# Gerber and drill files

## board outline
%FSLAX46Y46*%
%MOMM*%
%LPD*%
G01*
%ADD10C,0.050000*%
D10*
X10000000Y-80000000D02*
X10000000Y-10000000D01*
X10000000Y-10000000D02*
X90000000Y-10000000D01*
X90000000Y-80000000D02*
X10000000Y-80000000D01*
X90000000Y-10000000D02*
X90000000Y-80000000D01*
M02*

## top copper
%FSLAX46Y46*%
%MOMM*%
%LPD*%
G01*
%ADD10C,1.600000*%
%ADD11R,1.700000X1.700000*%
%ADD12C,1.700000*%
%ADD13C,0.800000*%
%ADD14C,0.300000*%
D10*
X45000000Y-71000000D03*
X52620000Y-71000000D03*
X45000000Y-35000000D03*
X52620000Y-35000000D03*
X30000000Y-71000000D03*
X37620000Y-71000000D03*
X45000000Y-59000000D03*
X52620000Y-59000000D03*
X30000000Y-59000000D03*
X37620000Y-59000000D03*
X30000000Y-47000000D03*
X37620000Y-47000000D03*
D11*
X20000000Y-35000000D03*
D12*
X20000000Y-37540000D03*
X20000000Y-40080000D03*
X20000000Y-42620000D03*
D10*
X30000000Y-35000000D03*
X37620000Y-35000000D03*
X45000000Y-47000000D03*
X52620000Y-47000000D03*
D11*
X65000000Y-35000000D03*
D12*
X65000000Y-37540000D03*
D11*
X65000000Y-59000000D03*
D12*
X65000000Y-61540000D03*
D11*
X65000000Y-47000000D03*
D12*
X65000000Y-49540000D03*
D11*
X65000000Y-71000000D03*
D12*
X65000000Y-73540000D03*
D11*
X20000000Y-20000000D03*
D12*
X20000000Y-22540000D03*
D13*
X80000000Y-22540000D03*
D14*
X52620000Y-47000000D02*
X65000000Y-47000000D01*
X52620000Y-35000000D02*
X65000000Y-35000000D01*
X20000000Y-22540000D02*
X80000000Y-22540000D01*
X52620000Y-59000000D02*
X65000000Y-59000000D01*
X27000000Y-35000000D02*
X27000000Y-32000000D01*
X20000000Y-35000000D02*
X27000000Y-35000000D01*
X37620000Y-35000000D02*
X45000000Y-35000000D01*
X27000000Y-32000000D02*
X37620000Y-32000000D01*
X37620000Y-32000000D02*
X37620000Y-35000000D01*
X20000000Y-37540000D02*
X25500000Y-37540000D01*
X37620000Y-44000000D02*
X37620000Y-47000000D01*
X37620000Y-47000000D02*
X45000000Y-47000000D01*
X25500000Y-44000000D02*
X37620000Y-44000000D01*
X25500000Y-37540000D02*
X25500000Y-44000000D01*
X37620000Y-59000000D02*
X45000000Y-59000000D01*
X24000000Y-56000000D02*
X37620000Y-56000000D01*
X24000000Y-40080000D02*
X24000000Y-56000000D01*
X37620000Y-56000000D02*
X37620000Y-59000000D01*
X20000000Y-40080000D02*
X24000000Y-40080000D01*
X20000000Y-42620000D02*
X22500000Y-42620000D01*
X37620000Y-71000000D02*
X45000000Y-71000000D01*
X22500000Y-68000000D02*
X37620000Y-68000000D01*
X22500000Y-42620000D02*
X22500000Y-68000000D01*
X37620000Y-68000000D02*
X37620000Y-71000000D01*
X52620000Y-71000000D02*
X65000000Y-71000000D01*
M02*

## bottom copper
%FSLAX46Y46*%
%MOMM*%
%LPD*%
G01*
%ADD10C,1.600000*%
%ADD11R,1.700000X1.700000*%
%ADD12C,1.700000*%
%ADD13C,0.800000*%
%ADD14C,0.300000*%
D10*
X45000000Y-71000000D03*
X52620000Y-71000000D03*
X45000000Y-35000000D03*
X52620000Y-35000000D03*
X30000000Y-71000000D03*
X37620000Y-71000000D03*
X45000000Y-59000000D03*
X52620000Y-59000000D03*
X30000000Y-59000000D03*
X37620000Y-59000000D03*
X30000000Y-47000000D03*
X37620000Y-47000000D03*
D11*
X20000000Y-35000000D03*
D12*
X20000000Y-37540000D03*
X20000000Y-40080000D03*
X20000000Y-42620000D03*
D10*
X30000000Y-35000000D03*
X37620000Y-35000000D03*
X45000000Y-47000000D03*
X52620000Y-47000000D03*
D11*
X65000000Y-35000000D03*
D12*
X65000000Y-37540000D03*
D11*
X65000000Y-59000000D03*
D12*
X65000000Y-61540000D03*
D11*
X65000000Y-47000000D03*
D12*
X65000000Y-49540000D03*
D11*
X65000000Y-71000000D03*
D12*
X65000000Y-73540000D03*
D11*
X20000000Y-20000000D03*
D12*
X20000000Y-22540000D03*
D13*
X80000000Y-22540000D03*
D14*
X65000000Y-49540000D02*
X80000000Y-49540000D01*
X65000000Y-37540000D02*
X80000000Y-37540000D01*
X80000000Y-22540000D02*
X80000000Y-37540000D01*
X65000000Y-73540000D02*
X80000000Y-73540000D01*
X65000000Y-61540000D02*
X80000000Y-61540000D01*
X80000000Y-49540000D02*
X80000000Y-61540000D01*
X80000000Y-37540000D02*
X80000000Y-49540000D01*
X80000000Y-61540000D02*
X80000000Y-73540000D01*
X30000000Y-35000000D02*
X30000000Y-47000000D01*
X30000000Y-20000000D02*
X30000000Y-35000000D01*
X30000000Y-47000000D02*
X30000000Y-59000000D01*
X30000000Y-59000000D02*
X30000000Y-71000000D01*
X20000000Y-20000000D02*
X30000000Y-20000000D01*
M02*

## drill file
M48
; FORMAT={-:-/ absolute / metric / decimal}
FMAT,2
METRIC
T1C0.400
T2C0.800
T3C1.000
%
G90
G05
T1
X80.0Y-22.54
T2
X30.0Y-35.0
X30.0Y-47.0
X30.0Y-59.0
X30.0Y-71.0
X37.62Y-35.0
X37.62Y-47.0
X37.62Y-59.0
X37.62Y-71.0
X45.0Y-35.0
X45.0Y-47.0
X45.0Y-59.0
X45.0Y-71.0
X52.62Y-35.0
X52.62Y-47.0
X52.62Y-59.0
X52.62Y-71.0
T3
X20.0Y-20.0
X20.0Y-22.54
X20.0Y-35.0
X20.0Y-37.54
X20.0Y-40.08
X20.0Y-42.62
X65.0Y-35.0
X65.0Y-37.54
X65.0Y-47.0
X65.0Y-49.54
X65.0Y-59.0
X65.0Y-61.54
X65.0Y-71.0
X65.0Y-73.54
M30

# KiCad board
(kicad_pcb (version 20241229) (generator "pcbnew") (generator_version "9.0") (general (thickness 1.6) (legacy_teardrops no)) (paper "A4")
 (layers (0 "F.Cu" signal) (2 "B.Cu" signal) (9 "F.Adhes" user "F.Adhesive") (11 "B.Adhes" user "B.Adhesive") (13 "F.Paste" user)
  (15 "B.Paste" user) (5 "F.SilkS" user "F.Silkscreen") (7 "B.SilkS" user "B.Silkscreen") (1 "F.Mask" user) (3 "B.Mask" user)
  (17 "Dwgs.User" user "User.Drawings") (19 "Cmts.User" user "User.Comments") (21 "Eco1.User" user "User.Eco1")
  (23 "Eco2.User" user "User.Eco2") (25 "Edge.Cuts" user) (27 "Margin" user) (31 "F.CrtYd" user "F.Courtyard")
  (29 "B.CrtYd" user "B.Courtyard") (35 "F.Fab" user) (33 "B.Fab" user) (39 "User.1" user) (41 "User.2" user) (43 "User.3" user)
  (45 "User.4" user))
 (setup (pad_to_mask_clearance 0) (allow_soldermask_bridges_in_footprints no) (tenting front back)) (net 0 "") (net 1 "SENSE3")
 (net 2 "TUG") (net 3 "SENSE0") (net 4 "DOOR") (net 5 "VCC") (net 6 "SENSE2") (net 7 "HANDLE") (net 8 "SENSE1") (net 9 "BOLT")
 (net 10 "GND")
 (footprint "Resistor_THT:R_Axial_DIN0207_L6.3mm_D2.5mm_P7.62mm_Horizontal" (layer "F.Cu") (at 45 71)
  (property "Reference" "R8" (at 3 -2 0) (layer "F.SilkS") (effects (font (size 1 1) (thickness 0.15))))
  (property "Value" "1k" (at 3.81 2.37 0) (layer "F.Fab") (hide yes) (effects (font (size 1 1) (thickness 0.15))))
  (pad "1" thru_hole circle (at 0 0) (size 1.6 1.6) (drill 0.8) (layers "*.Cu" "*.Mask") (remove_unused_layers no) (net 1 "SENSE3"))
  (pad "2" thru_hole circle (at 7.62 0) (size 1.6 1.6) (drill 0.8) (layers "*.Cu" "*.Mask") (remove_unused_layers no) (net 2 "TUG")))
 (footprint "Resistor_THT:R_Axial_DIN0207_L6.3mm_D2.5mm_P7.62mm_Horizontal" (layer "F.Cu") (at 45 35)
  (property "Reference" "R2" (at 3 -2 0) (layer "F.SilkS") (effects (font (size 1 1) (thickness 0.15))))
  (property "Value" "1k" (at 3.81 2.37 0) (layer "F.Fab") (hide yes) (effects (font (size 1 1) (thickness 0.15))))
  (pad "1" thru_hole circle (at 0 0) (size 1.6 1.6) (drill 0.8) (layers "*.Cu" "*.Mask") (remove_unused_layers no) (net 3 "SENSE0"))
  (pad "2" thru_hole circle (at 7.62 0) (size 1.6 1.6) (drill 0.8) (layers "*.Cu" "*.Mask") (remove_unused_layers no) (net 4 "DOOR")))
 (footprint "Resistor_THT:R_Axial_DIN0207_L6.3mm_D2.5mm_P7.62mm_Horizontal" (layer "F.Cu") (at 30 71)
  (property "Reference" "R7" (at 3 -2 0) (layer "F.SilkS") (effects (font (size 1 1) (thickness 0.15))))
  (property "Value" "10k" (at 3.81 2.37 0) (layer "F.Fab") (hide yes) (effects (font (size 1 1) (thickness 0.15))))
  (pad "1" thru_hole circle (at 0 0) (size 1.6 1.6) (drill 0.8) (layers "*.Cu" "*.Mask") (remove_unused_layers no) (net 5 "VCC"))
  (pad "2" thru_hole circle (at 7.62 0) (size 1.6 1.6) (drill 0.8) (layers "*.Cu" "*.Mask") (remove_unused_layers no) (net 1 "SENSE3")))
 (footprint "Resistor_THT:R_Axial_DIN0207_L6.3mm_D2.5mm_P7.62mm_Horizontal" (layer "F.Cu") (at 45 59)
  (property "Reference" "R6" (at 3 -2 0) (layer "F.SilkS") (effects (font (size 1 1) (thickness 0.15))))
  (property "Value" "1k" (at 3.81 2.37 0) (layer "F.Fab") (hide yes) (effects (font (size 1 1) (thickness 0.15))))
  (pad "1" thru_hole circle (at 0 0) (size 1.6 1.6) (drill 0.8) (layers "*.Cu" "*.Mask") (remove_unused_layers no) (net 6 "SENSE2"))
  (pad "2" thru_hole circle (at 7.62 0) (size 1.6 1.6) (drill 0.8) (layers "*.Cu" "*.Mask") (remove_unused_layers no) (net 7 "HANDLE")))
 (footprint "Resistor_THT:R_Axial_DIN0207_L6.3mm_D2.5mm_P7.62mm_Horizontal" (layer "F.Cu") (at 30 59)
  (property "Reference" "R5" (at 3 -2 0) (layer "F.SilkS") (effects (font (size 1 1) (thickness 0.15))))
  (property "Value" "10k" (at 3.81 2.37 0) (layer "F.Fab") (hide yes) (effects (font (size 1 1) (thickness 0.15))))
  (pad "1" thru_hole circle (at 0 0) (size 1.6 1.6) (drill 0.8) (layers "*.Cu" "*.Mask") (remove_unused_layers no) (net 5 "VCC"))
  (pad "2" thru_hole circle (at 7.62 0) (size 1.6 1.6) (drill 0.8) (layers "*.Cu" "*.Mask") (remove_unused_layers no) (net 6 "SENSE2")))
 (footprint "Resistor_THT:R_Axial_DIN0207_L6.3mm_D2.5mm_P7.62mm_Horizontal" (layer "F.Cu") (at 30 47)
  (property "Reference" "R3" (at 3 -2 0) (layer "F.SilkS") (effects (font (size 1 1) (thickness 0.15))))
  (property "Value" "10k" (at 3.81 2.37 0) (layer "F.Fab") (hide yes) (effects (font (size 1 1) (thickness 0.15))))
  (pad "1" thru_hole circle (at 0 0) (size 1.6 1.6) (drill 0.8) (layers "*.Cu" "*.Mask") (remove_unused_layers no) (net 5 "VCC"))
  (pad "2" thru_hole circle (at 7.62 0) (size 1.6 1.6) (drill 0.8) (layers "*.Cu" "*.Mask") (remove_unused_layers no) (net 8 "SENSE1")))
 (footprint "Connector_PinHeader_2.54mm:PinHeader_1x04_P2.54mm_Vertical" (layer "F.Cu") (at 20 35)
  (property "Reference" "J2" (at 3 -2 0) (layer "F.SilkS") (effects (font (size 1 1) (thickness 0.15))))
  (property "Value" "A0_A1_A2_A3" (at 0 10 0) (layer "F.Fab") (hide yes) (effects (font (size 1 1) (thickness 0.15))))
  (pad "1" thru_hole rect (at 0 0) (size 1.7 1.7) (drill 1) (layers "*.Cu" "*.Mask") (remove_unused_layers no) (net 3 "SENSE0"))
  (pad "2" thru_hole circle (at 0 2.54) (size 1.7 1.7) (drill 1) (layers "*.Cu" "*.Mask") (remove_unused_layers no) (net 8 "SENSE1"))
  (pad "3" thru_hole circle (at 0 5.08) (size 1.7 1.7) (drill 1) (layers "*.Cu" "*.Mask") (remove_unused_layers no) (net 6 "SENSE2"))
  (pad "4" thru_hole circle (at 0 7.62) (size 1.7 1.7) (drill 1) (layers "*.Cu" "*.Mask") (remove_unused_layers no) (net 1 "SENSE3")))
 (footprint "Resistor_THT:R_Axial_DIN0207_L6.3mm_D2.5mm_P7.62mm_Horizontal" (layer "F.Cu") (at 30 35)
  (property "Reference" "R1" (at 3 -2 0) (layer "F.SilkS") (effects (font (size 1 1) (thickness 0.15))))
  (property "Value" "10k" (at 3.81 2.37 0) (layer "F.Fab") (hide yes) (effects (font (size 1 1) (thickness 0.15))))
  (pad "1" thru_hole circle (at 0 0) (size 1.6 1.6) (drill 0.8) (layers "*.Cu" "*.Mask") (remove_unused_layers no) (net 5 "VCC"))
  (pad "2" thru_hole circle (at 7.62 0) (size 1.6 1.6) (drill 0.8) (layers "*.Cu" "*.Mask") (remove_unused_layers no) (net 3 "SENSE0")))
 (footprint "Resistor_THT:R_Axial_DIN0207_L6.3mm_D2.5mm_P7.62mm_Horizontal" (layer "F.Cu") (at 45 47)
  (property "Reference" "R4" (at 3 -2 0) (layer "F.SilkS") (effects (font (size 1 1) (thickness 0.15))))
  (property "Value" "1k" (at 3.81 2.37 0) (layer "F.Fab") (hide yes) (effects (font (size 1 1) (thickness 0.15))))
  (pad "1" thru_hole circle (at 0 0) (size 1.6 1.6) (drill 0.8) (layers "*.Cu" "*.Mask") (remove_unused_layers no) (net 8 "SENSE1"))
  (pad "2" thru_hole circle (at 7.62 0) (size 1.6 1.6) (drill 0.8) (layers "*.Cu" "*.Mask") (remove_unused_layers no) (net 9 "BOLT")))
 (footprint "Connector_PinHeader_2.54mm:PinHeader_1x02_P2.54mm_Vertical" (layer "F.Cu") (at 65 35)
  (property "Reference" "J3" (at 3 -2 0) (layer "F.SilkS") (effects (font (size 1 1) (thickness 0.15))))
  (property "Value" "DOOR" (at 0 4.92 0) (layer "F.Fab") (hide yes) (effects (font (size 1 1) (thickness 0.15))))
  (pad "1" thru_hole rect (at 0 0) (size 1.7 1.7) (drill 1) (layers "*.Cu" "*.Mask") (remove_unused_layers no) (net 4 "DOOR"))
  (pad "2" thru_hole circle (at 0 2.54) (size 1.7 1.7) (drill 1) (layers "*.Cu" "*.Mask") (remove_unused_layers no) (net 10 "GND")))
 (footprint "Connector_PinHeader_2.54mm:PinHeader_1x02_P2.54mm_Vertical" (layer "F.Cu") (at 65 59)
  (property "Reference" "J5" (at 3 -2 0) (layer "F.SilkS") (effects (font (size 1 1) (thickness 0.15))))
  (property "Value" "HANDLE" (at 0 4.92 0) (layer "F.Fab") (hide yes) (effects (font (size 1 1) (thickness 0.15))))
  (pad "1" thru_hole rect (at 0 0) (size 1.7 1.7) (drill 1) (layers "*.Cu" "*.Mask") (remove_unused_layers no) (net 7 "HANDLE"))
  (pad "2" thru_hole circle (at 0 2.54) (size 1.7 1.7) (drill 1) (layers "*.Cu" "*.Mask") (remove_unused_layers no) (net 10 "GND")))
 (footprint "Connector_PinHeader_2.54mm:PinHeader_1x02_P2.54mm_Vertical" (layer "F.Cu") (at 65 47)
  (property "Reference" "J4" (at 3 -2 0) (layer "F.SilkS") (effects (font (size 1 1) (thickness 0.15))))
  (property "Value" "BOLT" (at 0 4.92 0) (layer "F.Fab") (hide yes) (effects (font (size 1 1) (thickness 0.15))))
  (pad "1" thru_hole rect (at 0 0) (size 1.7 1.7) (drill 1) (layers "*.Cu" "*.Mask") (remove_unused_layers no) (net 9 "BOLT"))
  (pad "2" thru_hole circle (at 0 2.54) (size 1.7 1.7) (drill 1) (layers "*.Cu" "*.Mask") (remove_unused_layers no) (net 10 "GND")))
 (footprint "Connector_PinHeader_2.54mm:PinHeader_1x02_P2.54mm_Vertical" (layer "F.Cu") (at 65 71)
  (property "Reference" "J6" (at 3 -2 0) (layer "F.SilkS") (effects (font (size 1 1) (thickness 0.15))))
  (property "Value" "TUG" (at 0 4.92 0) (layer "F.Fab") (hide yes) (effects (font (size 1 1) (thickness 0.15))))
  (pad "1" thru_hole rect (at 0 0) (size 1.7 1.7) (drill 1) (layers "*.Cu" "*.Mask") (remove_unused_layers no) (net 2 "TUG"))
  (pad "2" thru_hole circle (at 0 2.54) (size 1.7 1.7) (drill 1) (layers "*.Cu" "*.Mask") (remove_unused_layers no) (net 10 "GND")))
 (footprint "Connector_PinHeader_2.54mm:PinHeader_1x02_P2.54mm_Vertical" (layer "F.Cu") (at 20 20)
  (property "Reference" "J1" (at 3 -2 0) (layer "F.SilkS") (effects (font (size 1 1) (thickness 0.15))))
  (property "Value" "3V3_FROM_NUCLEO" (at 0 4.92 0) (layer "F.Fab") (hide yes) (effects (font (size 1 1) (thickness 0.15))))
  (pad "1" thru_hole rect (at 0 0) (size 1.7 1.7) (drill 1) (layers "*.Cu" "*.Mask") (remove_unused_layers no) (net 5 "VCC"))
  (pad "2" thru_hole circle (at 0 2.54) (size 1.7 1.7) (drill 1) (layers "*.Cu" "*.Mask") (remove_unused_layers no) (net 10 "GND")))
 (gr_line (start 10 80) (end 10 10) (stroke (width 0.05) (type default)) (layer "Edge.Cuts"))
 (gr_line (start 10 10) (end 90 10) (stroke (width 0.05) (type default)) (layer "Edge.Cuts"))
 (gr_line (start 90 80) (end 10 80) (stroke (width 0.05) (type default)) (layer "Edge.Cuts"))
 (gr_line (start 90 10) (end 90 80) (stroke (width 0.05) (type default)) (layer "Edge.Cuts"))
 (segment (start 52.62 47) (end 65 47) (width 0.3) (layer "F.Cu") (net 9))
 (segment (start 52.62 35) (end 65 35) (width 0.3) (layer "F.Cu") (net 4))
 (segment (start 20 22.54) (end 80 22.54) (width 0.3) (layer "F.Cu") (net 10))
 (via (at 80 22.54) (size 0.8) (drill 0.4) (layers "F.Cu" "B.Cu") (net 10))
 (segment (start 65 49.54) (end 80 49.54) (width 0.3) (layer "B.Cu") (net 10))
 (segment (start 65 37.54) (end 80 37.54) (width 0.3) (layer "B.Cu") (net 10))
 (segment (start 80 22.54) (end 80 37.54) (width 0.3) (layer "B.Cu") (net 10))
 (segment (start 65 73.54) (end 80 73.54) (width 0.3) (layer "B.Cu") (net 10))
 (segment (start 65 61.54) (end 80 61.54) (width 0.3) (layer "B.Cu") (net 10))
 (segment (start 80 49.54) (end 80 61.54) (width 0.3) (layer "B.Cu") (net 10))
 (segment (start 80 37.54) (end 80 49.54) (width 0.3) (layer "B.Cu") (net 10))
 (segment (start 80 61.54) (end 80 73.54) (width 0.3) (layer "B.Cu") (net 10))
 (segment (start 52.62 59) (end 65 59) (width 0.3) (layer "F.Cu") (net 7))
 (segment (start 27 35) (end 27 32) (width 0.3) (layer "F.Cu") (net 3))
 (segment (start 20 35) (end 27 35) (width 0.3) (layer "F.Cu") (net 3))
 (segment (start 37.62 35) (end 45 35) (width 0.3) (layer "F.Cu") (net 3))
 (segment (start 27 32) (end 37.62 32) (width 0.3) (layer "F.Cu") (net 3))
 (segment (start 37.62 32) (end 37.62 35) (width 0.3) (layer "F.Cu") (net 3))
 (segment (start 20 37.54) (end 25.5 37.54) (width 0.3) (layer "F.Cu") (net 8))
 (segment (start 37.62 44) (end 37.62 47) (width 0.3) (layer "F.Cu") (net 8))
 (segment (start 37.62 47) (end 45 47) (width 0.3) (layer "F.Cu") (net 8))
 (segment (start 25.5 44) (end 37.62 44) (width 0.3) (layer "F.Cu") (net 8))
 (segment (start 25.5 37.54) (end 25.5 44) (width 0.3) (layer "F.Cu") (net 8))
 (segment (start 37.62 59) (end 45 59) (width 0.3) (layer "F.Cu") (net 6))
 (segment (start 24 56) (end 37.62 56) (width 0.3) (layer "F.Cu") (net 6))
 (segment (start 24 40.08) (end 24 56) (width 0.3) (layer "F.Cu") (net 6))
 (segment (start 37.62 56) (end 37.62 59) (width 0.3) (layer "F.Cu") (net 6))
 (segment (start 20 40.08) (end 24 40.08) (width 0.3) (layer "F.Cu") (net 6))
 (segment (start 20 42.62) (end 22.5 42.62) (width 0.3) (layer "F.Cu") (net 1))
 (segment (start 37.62 71) (end 45 71) (width 0.3) (layer "F.Cu") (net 1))
 (segment (start 22.5 68) (end 37.62 68) (width 0.3) (layer "F.Cu") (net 1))
 (segment (start 22.5 42.62) (end 22.5 68) (width 0.3) (layer "F.Cu") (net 1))
 (segment (start 37.62 68) (end 37.62 71) (width 0.3) (layer "F.Cu") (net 1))
 (segment (start 52.62 71) (end 65 71) (width 0.3) (layer "F.Cu") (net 2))
 (segment (start 30 35) (end 30 47) (width 0.3) (layer "B.Cu") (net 5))
 (segment (start 30 20) (end 30 35) (width 0.3) (layer "B.Cu") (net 5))
 (segment (start 30 47) (end 30 59) (width 0.3) (layer "B.Cu") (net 5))
 (segment (start 30 59) (end 30 71) (width 0.3) (layer "B.Cu") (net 5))
 (segment (start 20 20) (end 30 20) (width 0.3) (layer "B.Cu") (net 5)))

